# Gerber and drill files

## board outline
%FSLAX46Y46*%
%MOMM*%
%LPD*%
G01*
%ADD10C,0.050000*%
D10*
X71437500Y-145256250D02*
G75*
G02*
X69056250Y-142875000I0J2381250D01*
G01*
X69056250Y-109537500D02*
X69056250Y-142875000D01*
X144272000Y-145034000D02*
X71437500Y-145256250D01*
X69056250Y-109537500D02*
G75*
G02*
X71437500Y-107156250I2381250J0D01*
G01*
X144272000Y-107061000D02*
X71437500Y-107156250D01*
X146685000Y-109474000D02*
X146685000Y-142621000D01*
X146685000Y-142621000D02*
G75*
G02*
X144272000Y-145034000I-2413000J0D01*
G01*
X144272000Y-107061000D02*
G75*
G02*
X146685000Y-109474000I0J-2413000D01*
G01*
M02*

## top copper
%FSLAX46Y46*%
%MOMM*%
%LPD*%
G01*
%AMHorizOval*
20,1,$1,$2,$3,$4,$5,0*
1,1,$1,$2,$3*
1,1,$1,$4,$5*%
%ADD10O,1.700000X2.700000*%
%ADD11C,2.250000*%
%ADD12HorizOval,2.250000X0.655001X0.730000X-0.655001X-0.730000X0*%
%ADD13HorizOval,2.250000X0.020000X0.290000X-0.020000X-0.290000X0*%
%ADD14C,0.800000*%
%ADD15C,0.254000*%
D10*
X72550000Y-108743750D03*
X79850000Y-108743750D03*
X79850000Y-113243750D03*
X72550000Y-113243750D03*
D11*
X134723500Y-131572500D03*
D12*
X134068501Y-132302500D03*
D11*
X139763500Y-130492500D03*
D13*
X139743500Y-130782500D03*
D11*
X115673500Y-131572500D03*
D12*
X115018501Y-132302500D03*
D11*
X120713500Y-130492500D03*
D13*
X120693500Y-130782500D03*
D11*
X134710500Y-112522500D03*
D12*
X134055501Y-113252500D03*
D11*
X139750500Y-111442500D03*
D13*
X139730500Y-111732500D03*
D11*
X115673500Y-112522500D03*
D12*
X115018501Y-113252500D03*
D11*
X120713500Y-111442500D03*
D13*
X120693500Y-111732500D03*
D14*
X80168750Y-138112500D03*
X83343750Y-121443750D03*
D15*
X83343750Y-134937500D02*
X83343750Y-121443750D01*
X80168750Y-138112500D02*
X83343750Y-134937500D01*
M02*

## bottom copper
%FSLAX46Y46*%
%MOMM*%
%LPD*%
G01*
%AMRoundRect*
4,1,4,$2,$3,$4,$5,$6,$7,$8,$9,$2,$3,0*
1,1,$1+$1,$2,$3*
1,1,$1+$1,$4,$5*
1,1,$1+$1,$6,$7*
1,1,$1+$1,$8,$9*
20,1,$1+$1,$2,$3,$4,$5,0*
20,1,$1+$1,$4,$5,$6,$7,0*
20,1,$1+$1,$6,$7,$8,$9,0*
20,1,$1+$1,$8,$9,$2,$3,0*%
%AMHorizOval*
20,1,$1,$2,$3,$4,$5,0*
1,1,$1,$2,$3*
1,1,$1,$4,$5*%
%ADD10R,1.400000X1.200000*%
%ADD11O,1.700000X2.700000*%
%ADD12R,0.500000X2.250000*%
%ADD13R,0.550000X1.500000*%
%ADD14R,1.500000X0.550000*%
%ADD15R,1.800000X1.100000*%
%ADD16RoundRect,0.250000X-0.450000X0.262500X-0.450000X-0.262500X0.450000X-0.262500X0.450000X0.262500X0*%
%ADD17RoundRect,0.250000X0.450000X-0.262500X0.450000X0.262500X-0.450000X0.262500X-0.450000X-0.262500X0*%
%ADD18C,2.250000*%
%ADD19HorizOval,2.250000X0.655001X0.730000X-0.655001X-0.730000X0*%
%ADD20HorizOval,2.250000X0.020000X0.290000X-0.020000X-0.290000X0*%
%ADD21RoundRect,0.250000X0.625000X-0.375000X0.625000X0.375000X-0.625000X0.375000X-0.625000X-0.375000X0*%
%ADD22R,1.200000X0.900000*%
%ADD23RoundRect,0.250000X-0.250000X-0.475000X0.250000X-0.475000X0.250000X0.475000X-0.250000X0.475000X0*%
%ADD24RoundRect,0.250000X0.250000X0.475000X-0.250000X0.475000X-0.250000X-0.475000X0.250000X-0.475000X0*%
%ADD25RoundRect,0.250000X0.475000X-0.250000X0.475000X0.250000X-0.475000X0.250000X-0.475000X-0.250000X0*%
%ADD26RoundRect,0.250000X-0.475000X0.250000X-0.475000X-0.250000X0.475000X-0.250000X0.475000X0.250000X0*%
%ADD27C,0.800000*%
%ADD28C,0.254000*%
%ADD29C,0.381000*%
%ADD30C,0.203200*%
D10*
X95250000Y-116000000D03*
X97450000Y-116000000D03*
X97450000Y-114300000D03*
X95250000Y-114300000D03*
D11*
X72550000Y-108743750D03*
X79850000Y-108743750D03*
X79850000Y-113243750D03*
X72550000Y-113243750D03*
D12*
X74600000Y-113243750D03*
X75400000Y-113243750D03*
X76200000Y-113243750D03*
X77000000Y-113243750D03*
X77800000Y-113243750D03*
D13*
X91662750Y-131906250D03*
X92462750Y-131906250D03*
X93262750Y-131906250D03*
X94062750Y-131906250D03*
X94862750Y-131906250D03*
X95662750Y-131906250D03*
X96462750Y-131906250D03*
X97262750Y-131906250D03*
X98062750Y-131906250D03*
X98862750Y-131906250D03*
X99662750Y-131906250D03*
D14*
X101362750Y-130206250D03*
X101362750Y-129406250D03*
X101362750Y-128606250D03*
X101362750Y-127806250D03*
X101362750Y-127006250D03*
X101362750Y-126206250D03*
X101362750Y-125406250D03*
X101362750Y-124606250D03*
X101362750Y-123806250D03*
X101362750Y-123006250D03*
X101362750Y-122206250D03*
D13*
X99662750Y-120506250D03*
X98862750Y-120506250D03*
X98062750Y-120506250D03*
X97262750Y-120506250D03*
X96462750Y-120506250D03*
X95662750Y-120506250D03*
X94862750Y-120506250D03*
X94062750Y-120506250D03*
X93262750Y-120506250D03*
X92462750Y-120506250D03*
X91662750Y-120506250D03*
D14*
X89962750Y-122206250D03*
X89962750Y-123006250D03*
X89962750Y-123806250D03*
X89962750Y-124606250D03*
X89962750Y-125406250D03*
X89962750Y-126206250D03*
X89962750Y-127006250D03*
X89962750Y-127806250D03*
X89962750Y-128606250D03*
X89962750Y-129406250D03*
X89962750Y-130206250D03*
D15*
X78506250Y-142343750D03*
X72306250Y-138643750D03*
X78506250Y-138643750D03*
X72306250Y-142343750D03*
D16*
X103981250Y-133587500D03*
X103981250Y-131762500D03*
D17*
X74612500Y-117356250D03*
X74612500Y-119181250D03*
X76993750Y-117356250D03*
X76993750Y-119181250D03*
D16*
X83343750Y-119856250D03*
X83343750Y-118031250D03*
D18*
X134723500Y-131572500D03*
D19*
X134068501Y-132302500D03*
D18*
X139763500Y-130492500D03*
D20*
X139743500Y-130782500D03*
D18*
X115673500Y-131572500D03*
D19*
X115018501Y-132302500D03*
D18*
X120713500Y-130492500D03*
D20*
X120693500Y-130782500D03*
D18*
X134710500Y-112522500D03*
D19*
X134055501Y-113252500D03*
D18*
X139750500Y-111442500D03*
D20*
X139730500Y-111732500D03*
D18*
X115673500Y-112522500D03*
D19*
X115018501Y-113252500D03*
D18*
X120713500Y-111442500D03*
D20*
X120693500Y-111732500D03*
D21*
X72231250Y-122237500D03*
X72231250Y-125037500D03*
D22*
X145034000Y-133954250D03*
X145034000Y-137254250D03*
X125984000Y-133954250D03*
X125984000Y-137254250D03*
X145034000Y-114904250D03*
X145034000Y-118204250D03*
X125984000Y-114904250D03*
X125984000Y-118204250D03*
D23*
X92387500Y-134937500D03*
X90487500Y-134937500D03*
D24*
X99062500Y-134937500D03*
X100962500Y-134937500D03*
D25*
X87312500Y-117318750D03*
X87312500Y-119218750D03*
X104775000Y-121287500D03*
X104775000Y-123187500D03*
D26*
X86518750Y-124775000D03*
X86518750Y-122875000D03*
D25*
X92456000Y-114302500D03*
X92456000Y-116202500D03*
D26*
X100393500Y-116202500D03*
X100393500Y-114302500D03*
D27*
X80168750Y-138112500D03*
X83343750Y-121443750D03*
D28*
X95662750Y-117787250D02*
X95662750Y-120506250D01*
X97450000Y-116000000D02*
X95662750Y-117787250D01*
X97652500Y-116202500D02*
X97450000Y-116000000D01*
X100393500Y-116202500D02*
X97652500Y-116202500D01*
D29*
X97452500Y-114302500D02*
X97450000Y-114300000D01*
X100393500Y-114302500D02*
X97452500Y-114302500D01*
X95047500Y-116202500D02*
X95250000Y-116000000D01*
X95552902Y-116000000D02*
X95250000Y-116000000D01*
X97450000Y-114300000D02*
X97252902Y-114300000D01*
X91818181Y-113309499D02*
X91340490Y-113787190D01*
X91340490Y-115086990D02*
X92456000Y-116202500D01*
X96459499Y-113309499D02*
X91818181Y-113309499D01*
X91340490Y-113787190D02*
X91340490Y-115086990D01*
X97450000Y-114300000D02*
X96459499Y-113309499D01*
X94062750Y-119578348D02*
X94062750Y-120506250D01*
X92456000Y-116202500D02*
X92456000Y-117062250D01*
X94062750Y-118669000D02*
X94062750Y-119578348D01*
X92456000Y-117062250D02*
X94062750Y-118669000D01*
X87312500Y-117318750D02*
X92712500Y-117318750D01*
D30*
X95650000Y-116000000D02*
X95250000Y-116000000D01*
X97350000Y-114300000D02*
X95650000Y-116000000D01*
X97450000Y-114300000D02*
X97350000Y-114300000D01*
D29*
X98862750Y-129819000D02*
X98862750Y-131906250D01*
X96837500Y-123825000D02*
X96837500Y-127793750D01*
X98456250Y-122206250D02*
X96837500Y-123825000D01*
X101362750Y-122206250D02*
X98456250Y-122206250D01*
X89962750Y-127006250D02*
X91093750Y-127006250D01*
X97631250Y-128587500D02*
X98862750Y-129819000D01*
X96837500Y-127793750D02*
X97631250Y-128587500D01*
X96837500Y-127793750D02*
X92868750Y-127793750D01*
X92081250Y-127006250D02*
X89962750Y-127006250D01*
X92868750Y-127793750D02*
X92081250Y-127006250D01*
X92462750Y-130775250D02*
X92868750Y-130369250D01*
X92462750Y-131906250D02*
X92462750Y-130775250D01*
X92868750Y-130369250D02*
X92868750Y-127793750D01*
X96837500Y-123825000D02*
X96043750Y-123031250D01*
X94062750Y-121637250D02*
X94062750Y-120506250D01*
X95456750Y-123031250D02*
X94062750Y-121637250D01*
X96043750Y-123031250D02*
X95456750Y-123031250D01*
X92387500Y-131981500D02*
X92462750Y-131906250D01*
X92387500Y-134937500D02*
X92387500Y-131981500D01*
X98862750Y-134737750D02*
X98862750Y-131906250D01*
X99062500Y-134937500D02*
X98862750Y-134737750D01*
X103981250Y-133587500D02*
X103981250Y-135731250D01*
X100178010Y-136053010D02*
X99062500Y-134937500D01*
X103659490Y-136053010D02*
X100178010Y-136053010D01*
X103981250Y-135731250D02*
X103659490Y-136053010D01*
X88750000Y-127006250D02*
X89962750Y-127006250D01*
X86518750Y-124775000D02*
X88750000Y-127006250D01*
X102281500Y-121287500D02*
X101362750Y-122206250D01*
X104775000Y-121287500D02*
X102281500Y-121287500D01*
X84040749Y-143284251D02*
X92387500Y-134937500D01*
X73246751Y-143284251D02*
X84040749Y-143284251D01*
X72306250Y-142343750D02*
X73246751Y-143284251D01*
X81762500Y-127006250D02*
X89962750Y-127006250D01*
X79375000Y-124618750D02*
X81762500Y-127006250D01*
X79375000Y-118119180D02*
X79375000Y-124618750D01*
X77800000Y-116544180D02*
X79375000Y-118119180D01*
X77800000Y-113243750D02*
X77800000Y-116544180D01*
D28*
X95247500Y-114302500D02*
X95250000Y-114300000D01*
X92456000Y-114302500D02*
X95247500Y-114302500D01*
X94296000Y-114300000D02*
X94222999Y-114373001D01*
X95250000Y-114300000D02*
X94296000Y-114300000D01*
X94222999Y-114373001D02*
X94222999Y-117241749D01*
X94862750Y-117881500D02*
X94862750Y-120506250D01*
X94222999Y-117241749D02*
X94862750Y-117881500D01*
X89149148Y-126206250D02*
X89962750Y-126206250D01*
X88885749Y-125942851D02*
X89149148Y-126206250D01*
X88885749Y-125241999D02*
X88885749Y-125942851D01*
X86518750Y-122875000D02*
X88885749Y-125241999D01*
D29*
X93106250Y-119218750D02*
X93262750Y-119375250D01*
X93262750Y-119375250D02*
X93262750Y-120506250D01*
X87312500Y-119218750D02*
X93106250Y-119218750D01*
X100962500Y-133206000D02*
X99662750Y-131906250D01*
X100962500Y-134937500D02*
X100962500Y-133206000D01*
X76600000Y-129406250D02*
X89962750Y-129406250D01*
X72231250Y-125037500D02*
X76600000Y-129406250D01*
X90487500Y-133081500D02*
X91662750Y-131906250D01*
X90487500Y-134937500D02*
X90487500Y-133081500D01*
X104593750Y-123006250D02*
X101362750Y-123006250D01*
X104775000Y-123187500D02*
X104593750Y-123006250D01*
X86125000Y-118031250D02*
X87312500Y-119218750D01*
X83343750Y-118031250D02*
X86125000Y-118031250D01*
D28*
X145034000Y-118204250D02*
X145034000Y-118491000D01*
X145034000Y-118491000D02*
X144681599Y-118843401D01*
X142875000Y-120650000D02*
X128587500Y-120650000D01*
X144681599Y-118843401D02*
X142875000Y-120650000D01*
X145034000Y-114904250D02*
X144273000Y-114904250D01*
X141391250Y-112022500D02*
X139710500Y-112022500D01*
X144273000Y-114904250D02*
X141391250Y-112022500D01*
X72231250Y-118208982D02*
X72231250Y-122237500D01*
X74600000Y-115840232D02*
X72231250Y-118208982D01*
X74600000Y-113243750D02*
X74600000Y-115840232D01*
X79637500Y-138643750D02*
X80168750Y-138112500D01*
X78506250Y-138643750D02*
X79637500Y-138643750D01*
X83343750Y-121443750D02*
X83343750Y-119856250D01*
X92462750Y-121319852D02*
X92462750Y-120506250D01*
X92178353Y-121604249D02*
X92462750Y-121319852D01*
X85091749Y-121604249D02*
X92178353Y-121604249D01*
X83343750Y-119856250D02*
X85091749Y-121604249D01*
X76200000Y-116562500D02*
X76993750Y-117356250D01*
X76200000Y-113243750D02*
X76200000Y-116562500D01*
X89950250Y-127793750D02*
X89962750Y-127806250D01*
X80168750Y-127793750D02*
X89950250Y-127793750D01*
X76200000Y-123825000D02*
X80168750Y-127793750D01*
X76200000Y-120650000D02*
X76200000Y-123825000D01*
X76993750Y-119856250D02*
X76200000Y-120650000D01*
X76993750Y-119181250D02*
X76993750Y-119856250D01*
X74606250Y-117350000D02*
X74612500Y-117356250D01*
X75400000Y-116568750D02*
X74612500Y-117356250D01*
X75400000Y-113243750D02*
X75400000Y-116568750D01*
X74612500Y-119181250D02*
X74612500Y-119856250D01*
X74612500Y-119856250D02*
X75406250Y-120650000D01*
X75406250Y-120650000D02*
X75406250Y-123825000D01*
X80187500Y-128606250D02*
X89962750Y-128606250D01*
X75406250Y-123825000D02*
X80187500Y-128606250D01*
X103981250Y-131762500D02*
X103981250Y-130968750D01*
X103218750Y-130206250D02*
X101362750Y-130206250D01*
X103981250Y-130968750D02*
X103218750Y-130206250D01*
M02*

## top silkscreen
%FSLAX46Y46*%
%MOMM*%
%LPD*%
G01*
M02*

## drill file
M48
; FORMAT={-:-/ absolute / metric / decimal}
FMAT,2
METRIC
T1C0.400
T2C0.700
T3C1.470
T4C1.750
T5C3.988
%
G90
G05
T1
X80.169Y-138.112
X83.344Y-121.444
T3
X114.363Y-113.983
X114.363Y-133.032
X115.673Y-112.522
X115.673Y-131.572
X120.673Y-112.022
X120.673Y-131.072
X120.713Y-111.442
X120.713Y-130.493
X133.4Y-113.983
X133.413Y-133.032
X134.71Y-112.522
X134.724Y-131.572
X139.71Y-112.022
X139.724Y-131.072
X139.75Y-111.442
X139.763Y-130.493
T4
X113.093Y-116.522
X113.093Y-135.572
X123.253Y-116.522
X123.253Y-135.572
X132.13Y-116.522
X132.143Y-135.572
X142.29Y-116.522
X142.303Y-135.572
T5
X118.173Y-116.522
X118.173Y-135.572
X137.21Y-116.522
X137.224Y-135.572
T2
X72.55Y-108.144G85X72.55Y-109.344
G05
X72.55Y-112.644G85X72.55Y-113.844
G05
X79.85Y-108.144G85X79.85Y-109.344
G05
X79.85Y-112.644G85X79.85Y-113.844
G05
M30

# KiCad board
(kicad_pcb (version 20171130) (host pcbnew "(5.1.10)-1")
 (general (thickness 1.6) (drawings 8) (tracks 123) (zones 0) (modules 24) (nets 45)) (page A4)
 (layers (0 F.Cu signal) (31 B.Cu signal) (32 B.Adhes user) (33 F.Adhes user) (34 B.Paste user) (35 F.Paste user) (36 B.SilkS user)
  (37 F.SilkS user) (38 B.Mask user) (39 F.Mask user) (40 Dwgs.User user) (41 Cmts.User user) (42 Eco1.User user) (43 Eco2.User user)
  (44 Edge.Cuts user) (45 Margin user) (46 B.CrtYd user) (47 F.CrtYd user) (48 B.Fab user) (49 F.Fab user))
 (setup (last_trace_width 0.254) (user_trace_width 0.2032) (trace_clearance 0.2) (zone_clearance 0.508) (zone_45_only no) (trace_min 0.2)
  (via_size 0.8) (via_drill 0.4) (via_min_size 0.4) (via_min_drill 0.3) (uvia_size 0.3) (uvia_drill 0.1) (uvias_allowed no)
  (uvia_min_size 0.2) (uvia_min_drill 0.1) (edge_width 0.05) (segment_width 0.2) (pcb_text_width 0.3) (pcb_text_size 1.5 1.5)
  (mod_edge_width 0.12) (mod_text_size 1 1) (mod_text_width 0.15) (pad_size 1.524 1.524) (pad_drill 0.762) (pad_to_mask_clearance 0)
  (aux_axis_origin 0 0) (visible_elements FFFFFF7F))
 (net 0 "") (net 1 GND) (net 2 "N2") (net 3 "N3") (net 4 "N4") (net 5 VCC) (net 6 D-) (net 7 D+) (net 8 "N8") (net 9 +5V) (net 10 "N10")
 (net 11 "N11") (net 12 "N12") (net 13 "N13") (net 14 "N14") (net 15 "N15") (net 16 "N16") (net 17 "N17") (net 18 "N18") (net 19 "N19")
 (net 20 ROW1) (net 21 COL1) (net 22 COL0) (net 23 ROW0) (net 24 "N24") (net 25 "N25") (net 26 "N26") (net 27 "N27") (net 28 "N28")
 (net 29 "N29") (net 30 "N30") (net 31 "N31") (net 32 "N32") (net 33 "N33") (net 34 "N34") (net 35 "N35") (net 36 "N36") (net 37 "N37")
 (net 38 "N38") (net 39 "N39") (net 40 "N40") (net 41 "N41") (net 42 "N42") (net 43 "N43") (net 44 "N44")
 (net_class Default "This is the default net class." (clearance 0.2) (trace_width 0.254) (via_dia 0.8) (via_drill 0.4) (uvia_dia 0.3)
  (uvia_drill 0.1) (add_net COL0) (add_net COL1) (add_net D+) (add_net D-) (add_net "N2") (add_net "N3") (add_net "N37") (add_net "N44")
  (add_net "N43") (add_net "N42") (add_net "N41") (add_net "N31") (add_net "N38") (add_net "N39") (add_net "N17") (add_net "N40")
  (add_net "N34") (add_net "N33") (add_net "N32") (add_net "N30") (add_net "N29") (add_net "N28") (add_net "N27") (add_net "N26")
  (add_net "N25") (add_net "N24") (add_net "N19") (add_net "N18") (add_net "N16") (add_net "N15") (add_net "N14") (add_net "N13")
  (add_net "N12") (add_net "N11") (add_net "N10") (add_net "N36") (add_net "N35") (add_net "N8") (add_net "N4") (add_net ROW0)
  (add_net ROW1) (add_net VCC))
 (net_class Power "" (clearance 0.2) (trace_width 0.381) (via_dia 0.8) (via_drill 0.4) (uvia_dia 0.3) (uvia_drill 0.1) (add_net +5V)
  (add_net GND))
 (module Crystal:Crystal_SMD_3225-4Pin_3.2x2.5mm (layer B.Cu) (at 96.35 115.15)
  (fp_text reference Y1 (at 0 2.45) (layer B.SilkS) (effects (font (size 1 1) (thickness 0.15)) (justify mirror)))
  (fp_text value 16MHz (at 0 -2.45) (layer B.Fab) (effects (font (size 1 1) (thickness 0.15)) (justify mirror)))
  (pad 4 smd rect (at -1.1 0.85) (size 1.4 1.2) (layers B.Cu B.Paste B.Mask) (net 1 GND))
  (pad 3 smd rect (at 1.1 0.85) (size 1.4 1.2) (layers B.Cu B.Paste B.Mask) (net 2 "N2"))
  (pad 2 smd rect (at 1.1 -0.85) (size 1.4 1.2) (layers B.Cu B.Paste B.Mask) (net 1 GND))
  (pad 1 smd rect (at -1.1 -0.85) (size 1.4 1.2) (layers B.Cu B.Paste B.Mask) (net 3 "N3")))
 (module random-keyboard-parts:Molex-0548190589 (layer B.Cu) (at 76.2 108.74375 270)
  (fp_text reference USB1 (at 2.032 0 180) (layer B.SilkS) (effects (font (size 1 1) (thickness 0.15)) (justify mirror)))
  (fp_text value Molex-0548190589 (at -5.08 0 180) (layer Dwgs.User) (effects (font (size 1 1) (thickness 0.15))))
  (pad 6 thru_hole oval (at 0 3.65 270) (size 2.7 1.7) (drill oval 1.9 0.7) (layers *.Cu *.Mask) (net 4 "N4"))
  (pad 6 thru_hole oval (at 0 -3.65 270) (size 2.7 1.7) (drill oval 1.9 0.7) (layers *.Cu *.Mask) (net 4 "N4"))
  (pad 6 thru_hole oval (at 4.5 -3.65 270) (size 2.7 1.7) (drill oval 1.9 0.7) (layers *.Cu *.Mask) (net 4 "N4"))
  (pad 6 thru_hole oval (at 4.5 3.65 270) (size 2.7 1.7) (drill oval 1.9 0.7) (layers *.Cu *.Mask) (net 4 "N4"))
  (pad 5 smd rect (at 4.5 1.6 270) (size 2.25 0.5) (layers B.Cu B.Paste B.Mask) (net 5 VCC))
  (pad 4 smd rect (at 4.5 0.8 270) (size 2.25 0.5) (layers B.Cu B.Paste B.Mask) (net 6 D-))
  (pad 3 smd rect (at 4.5 0 270) (size 2.25 0.5) (layers B.Cu B.Paste B.Mask) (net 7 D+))
  (pad 2 smd rect (at 4.5 -0.8 270) (size 2.25 0.5) (layers B.Cu B.Paste B.Mask) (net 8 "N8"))
  (pad 1 smd rect (at 4.5 -1.6 270) (size 2.25 0.5) (layers B.Cu B.Paste B.Mask) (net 1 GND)))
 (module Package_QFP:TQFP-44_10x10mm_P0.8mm (layer B.Cu) (at 95.66275 126.20625)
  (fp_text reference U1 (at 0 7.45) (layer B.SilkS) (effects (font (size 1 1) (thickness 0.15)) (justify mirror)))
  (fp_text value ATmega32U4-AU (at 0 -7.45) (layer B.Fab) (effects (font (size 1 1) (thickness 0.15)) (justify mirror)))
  (pad 44 smd rect (at -4 5.7 270) (size 1.5 0.55) (layers B.Cu B.Paste B.Mask) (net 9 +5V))
  (pad 43 smd rect (at -3.2 5.7 270) (size 1.5 0.55) (layers B.Cu B.Paste B.Mask) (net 1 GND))
  (pad 42 smd rect (at -2.4 5.7 270) (size 1.5 0.55) (layers B.Cu B.Paste B.Mask) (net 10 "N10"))
  (pad 41 smd rect (at -1.6 5.7 270) (size 1.5 0.55) (layers B.Cu B.Paste B.Mask) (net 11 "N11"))
  (pad 40 smd rect (at -0.8 5.7 270) (size 1.5 0.55) (layers B.Cu B.Paste B.Mask) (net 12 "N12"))
  (pad 39 smd rect (at 0 5.7 270) (size 1.5 0.55) (layers B.Cu B.Paste B.Mask) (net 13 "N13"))
  (pad 38 smd rect (at 0.8 5.7 270) (size 1.5 0.55) (layers B.Cu B.Paste B.Mask) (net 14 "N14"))
  (pad 37 smd rect (at 1.6 5.7 270) (size 1.5 0.55) (layers B.Cu B.Paste B.Mask) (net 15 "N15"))
  (pad 36 smd rect (at 2.4 5.7 270) (size 1.5 0.55) (layers B.Cu B.Paste B.Mask) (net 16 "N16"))
  (pad 35 smd rect (at 3.2 5.7 270) (size 1.5 0.55) (layers B.Cu B.Paste B.Mask) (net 1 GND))
  (pad 34 smd rect (at 4 5.7 270) (size 1.5 0.55) (layers B.Cu B.Paste B.Mask) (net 9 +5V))
  (pad 33 smd rect (at 5.7 4) (size 1.5 0.55) (layers B.Cu B.Paste B.Mask) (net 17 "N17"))
  (pad 32 smd rect (at 5.7 3.2) (size 1.5 0.55) (layers B.Cu B.Paste B.Mask) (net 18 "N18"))
  (pad 31 smd rect (at 5.7 2.4) (size 1.5 0.55) (layers B.Cu B.Paste B.Mask) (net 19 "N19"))
  (pad 30 smd rect (at 5.7 1.6) (size 1.5 0.55) (layers B.Cu B.Paste B.Mask) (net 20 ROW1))
  (pad 29 smd rect (at 5.7 0.8) (size 1.5 0.55) (layers B.Cu B.Paste B.Mask) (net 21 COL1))
  (pad 28 smd rect (at 5.7 0) (size 1.5 0.55) (layers B.Cu B.Paste B.Mask) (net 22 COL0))
  (pad 27 smd rect (at 5.7 -0.8) (size 1.5 0.55) (layers B.Cu B.Paste B.Mask) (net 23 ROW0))
  (pad 26 smd rect (at 5.7 -1.6) (size 1.5 0.55) (layers B.Cu B.Paste B.Mask) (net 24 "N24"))
  (pad 25 smd rect (at 5.7 -2.4) (size 1.5 0.55) (layers B.Cu B.Paste B.Mask) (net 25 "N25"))
  (pad 24 smd rect (at 5.7 -3.2) (size 1.5 0.55) (layers B.Cu B.Paste B.Mask) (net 9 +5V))
  (pad 23 smd rect (at 5.7 -4) (size 1.5 0.55) (layers B.Cu B.Paste B.Mask) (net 1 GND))
  (pad 22 smd rect (at 4 -5.7 270) (size 1.5 0.55) (layers B.Cu B.Paste B.Mask) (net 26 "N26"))
  (pad 21 smd rect (at 3.2 -5.7 270) (size 1.5 0.55) (layers B.Cu B.Paste B.Mask) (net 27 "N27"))
  (pad 20 smd rect (at 2.4 -5.7 270) (size 1.5 0.55) (layers B.Cu B.Paste B.Mask) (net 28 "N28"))
  (pad 19 smd rect (at 1.6 -5.7 270) (size 1.5 0.55) (layers B.Cu B.Paste B.Mask) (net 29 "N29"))
  (pad 18 smd rect (at 0.8 -5.7 270) (size 1.5 0.55) (layers B.Cu B.Paste B.Mask) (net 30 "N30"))
  (pad 17 smd rect (at 0 -5.7 270) (size 1.5 0.55) (layers B.Cu B.Paste B.Mask) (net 2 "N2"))
  (pad 16 smd rect (at -0.8 -5.7 270) (size 1.5 0.55) (layers B.Cu B.Paste B.Mask) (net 3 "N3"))
  (pad 15 smd rect (at -1.6 -5.7 270) (size 1.5 0.55) (layers B.Cu B.Paste B.Mask) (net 1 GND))
  (pad 14 smd rect (at -2.4 -5.7 270) (size 1.5 0.55) (layers B.Cu B.Paste B.Mask) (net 9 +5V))
  (pad 13 smd rect (at -3.2 -5.7 270) (size 1.5 0.55) (layers B.Cu B.Paste B.Mask) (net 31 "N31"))
  (pad 12 smd rect (at -4 -5.7 270) (size 1.5 0.55) (layers B.Cu B.Paste B.Mask) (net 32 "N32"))
  (pad 11 smd rect (at -5.7 -4) (size 1.5 0.55) (layers B.Cu B.Paste B.Mask) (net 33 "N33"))
  (pad 10 smd rect (at -5.7 -3.2) (size 1.5 0.55) (layers B.Cu B.Paste B.Mask) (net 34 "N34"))
  (pad 9 smd rect (at -5.7 -2.4) (size 1.5 0.55) (layers B.Cu B.Paste B.Mask) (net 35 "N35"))
  (pad 8 smd rect (at -5.7 -1.6) (size 1.5 0.55) (layers B.Cu B.Paste B.Mask) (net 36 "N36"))
  (pad 7 smd rect (at -5.7 -0.8) (size 1.5 0.55) (layers B.Cu B.Paste B.Mask) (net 9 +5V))
  (pad 6 smd rect (at -5.7 0) (size 1.5 0.55) (layers B.Cu B.Paste B.Mask) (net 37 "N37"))
  (pad 5 smd rect (at -5.7 0.8) (size 1.5 0.55) (layers B.Cu B.Paste B.Mask) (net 1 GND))
  (pad 4 smd rect (at -5.7 1.6) (size 1.5 0.55) (layers B.Cu B.Paste B.Mask) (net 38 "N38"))
  (pad 3 smd rect (at -5.7 2.4) (size 1.5 0.55) (layers B.Cu B.Paste B.Mask) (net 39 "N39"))
  (pad 2 smd rect (at -5.7 3.2) (size 1.5 0.55) (layers B.Cu B.Paste B.Mask) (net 9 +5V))
  (pad 1 smd rect (at -5.7 4) (size 1.5 0.55) (layers B.Cu B.Paste B.Mask) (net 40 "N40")))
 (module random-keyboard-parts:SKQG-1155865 (layer B.Cu) (at 75.40625 140.49375 180)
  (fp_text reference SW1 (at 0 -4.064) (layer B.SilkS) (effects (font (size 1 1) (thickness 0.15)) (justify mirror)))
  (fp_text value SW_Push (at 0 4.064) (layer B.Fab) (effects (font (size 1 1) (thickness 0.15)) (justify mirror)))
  (pad 4 smd rect (at -3.1 -1.85 180) (size 1.8 1.1) (layers B.Cu B.Paste B.Mask))
  (pad 3 smd rect (at 3.1 1.85 180) (size 1.8 1.1) (layers B.Cu B.Paste B.Mask))
  (pad 2 smd rect (at -3.1 1.85 180) (size 1.8 1.1) (layers B.Cu B.Paste B.Mask) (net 31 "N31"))
  (pad 1 smd rect (at 3.1 -1.85 180) (size 1.8 1.1) (layers B.Cu B.Paste B.Mask) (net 1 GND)))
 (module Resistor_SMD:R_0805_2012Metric (layer B.Cu) (at 103.98125 132.675 270)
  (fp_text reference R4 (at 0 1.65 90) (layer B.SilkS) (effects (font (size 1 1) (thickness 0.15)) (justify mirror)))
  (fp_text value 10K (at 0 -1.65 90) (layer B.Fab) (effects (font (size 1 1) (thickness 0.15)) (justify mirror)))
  (pad 2 smd roundrect (at 0.9125 0 270) (size 1.025 1.4) (layers B.Cu B.Paste B.Mask) (roundrect_rratio 0.243902) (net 1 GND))
  (pad 1 smd roundrect (at -0.9125 0 270) (size 1.025 1.4) (layers B.Cu B.Paste B.Mask) (roundrect_rratio 0.243902) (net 17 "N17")))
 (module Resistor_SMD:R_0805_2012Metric (layer B.Cu) (at 74.6125 118.26875 90)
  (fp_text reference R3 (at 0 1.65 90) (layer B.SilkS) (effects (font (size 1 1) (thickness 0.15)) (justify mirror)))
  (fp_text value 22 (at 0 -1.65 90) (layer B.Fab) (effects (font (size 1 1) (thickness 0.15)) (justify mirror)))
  (pad 2 smd roundrect (at 0.9125 0 90) (size 1.025 1.4) (layers B.Cu B.Paste B.Mask) (roundrect_rratio 0.243902) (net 6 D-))
  (pad 1 smd roundrect (at -0.9125 0 90) (size 1.025 1.4) (layers B.Cu B.Paste B.Mask) (roundrect_rratio 0.243902) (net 39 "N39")))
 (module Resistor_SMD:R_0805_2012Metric (layer B.Cu) (at 76.99375 118.26875 90)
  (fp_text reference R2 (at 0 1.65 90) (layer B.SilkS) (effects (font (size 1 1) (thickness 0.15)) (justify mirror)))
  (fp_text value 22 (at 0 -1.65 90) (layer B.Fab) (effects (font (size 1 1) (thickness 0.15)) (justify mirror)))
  (pad 2 smd roundrect (at 0.9125 0 90) (size 1.025 1.4) (layers B.Cu B.Paste B.Mask) (roundrect_rratio 0.243902) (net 7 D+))
  (pad 1 smd roundrect (at -0.9125 0 90) (size 1.025 1.4) (layers B.Cu B.Paste B.Mask) (roundrect_rratio 0.243902) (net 38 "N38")))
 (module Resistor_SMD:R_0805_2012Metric (layer B.Cu) (at 83.34375 118.94375 270)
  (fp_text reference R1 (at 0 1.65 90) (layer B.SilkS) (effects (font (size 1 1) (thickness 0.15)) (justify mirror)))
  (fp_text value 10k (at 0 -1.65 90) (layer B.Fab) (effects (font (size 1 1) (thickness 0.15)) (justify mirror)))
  (pad 2 smd roundrect (at 0.9125 0 270) (size 1.025 1.4) (layers B.Cu B.Paste B.Mask) (roundrect_rratio 0.243902) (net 31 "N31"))
  (pad 1 smd roundrect (at -0.9125 0 270) (size 1.025 1.4) (layers B.Cu B.Paste B.Mask) (roundrect_rratio 0.243902) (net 9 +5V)))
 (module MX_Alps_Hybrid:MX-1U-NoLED (layer F.Cu) (at 137.2235 135.5725)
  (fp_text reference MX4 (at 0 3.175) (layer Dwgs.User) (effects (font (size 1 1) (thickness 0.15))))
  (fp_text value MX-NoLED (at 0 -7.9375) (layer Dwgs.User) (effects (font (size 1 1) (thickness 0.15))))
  (pad "" np_thru_hole circle (at 5.08 0 48.0996) (size 1.75 1.75) (drill 1.75) (layers *.Cu *.Mask))
  (pad "" np_thru_hole circle (at -5.08 0 48.0996) (size 1.75 1.75) (drill 1.75) (layers *.Cu *.Mask))
  (pad 1 thru_hole circle (at -2.5 -4) (size 2.25 2.25) (drill 1.47) (layers *.Cu B.Mask) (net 21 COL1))
  (pad "" np_thru_hole circle (at 0 0) (size 3.9878 3.9878) (drill 3.9878) (layers *.Cu *.Mask))
  (pad 1 thru_hole oval (at -3.81 -2.54 48.0996) (size 4.211556 2.25) (drill 1.47 (offset 0.980778 0)) (layers *.Cu B.Mask) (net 21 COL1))
  (pad 2 thru_hole circle (at 2.54 -5.08) (size 2.25 2.25) (drill 1.47) (layers *.Cu B.Mask) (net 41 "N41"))
  (pad 2 thru_hole oval (at 2.5 -4.5 86.0548) (size 2.831378 2.25) (drill 1.47 (offset 0.290689 0)) (layers *.Cu B.Mask) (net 41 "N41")))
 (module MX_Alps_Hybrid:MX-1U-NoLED (layer F.Cu) (at 118.1735 135.5725)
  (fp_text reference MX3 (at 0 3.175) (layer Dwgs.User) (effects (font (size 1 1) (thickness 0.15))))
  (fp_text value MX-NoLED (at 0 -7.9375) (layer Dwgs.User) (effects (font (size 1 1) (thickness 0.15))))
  (pad "" np_thru_hole circle (at 5.08 0 48.0996) (size 1.75 1.75) (drill 1.75) (layers *.Cu *.Mask))
  (pad "" np_thru_hole circle (at -5.08 0 48.0996) (size 1.75 1.75) (drill 1.75) (layers *.Cu *.Mask))
  (pad 1 thru_hole circle (at -2.5 -4) (size 2.25 2.25) (drill 1.47) (layers *.Cu B.Mask) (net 22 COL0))
  (pad "" np_thru_hole circle (at 0 0) (size 3.9878 3.9878) (drill 3.9878) (layers *.Cu *.Mask))
  (pad 1 thru_hole oval (at -3.81 -2.54 48.0996) (size 4.211556 2.25) (drill 1.47 (offset 0.980778 0)) (layers *.Cu B.Mask) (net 22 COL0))
  (pad 2 thru_hole circle (at 2.54 -5.08) (size 2.25 2.25) (drill 1.47) (layers *.Cu B.Mask) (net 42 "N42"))
  (pad 2 thru_hole oval (at 2.5 -4.5 86.0548) (size 2.831378 2.25) (drill 1.47 (offset 0.290689 0)) (layers *.Cu B.Mask) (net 42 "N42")))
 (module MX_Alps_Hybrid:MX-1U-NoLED (layer F.Cu) (at 137.2105 116.5225)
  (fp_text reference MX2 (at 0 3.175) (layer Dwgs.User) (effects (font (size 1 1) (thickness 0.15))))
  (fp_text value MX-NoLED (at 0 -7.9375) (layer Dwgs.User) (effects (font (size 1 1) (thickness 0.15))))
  (pad "" np_thru_hole circle (at 5.08 0 48.0996) (size 1.75 1.75) (drill 1.75) (layers *.Cu *.Mask))
  (pad "" np_thru_hole circle (at -5.08 0 48.0996) (size 1.75 1.75) (drill 1.75) (layers *.Cu *.Mask))
  (pad 1 thru_hole circle (at -2.5 -4) (size 2.25 2.25) (drill 1.47) (layers *.Cu B.Mask) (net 21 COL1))
  (pad "" np_thru_hole circle (at 0 0) (size 3.9878 3.9878) (drill 3.9878) (layers *.Cu *.Mask))
  (pad 1 thru_hole oval (at -3.81 -2.54 48.0996) (size 4.211556 2.25) (drill 1.47 (offset 0.980778 0)) (layers *.Cu B.Mask) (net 21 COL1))
  (pad 2 thru_hole circle (at 2.54 -5.08) (size 2.25 2.25) (drill 1.47) (layers *.Cu B.Mask) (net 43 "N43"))
  (pad 2 thru_hole oval (at 2.5 -4.5 86.0548) (size 2.831378 2.25) (drill 1.47 (offset 0.290689 0)) (layers *.Cu B.Mask) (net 43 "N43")))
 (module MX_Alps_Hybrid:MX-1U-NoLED (layer F.Cu) (at 118.1735 116.5225)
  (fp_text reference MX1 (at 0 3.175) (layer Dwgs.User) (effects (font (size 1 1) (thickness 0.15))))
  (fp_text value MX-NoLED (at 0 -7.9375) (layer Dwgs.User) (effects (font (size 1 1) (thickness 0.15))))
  (pad "" np_thru_hole circle (at 5.08 0 48.0996) (size 1.75 1.75) (drill 1.75) (layers *.Cu *.Mask))
  (pad "" np_thru_hole circle (at -5.08 0 48.0996) (size 1.75 1.75) (drill 1.75) (layers *.Cu *.Mask))
  (pad 1 thru_hole circle (at -2.5 -4) (size 2.25 2.25) (drill 1.47) (layers *.Cu B.Mask) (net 22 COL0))
  (pad "" np_thru_hole circle (at 0 0) (size 3.9878 3.9878) (drill 3.9878) (layers *.Cu *.Mask))
  (pad 1 thru_hole oval (at -3.81 -2.54 48.0996) (size 4.211556 2.25) (drill 1.47 (offset 0.980778 0)) (layers *.Cu B.Mask) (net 22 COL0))
  (pad 2 thru_hole circle (at 2.54 -5.08) (size 2.25 2.25) (drill 1.47) (layers *.Cu B.Mask) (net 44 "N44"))
  (pad 2 thru_hole oval (at 2.5 -4.5 86.0548) (size 2.831378 2.25) (drill 1.47 (offset 0.290689 0)) (layers *.Cu B.Mask) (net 44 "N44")))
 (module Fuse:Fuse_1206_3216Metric (layer B.Cu) (at 72.23125 123.6375 90)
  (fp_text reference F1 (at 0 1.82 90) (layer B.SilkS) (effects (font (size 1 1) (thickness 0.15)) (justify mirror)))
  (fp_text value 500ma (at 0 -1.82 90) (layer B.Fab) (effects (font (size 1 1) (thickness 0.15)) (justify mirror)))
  (pad 2 smd roundrect (at 1.4 0 90) (size 1.25 1.75) (layers B.Cu B.Paste B.Mask) (roundrect_rratio 0.2) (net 5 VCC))
  (pad 1 smd roundrect (at -1.4 0 90) (size 1.25 1.75) (layers B.Cu B.Paste B.Mask) (roundrect_rratio 0.2) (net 9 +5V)))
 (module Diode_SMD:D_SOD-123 (layer B.Cu) (at 145.034 135.60425 90)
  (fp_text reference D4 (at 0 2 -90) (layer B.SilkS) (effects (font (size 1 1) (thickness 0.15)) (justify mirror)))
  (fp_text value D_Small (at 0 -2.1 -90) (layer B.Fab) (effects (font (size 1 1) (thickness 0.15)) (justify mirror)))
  (pad 2 smd rect (at 1.65 0 90) (size 0.9 1.2) (layers B.Cu B.Paste B.Mask) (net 41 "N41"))
  (pad 1 smd rect (at -1.65 0 90) (size 0.9 1.2) (layers B.Cu B.Paste B.Mask) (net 20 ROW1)))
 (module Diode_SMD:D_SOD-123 (layer B.Cu) (at 125.984 135.60425 90)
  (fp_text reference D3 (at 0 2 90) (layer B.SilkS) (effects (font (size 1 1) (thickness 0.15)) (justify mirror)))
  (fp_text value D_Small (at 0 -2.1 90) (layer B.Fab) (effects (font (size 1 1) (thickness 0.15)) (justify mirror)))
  (pad 2 smd rect (at 1.65 0 90) (size 0.9 1.2) (layers B.Cu B.Paste B.Mask) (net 42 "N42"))
  (pad 1 smd rect (at -1.65 0 90) (size 0.9 1.2) (layers B.Cu B.Paste B.Mask) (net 20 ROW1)))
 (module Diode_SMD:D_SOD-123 (layer B.Cu) (at 145.034 116.55425 90)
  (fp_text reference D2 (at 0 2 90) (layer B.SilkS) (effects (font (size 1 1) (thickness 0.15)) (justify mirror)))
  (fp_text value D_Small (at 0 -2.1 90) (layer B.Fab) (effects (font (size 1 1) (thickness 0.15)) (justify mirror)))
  (pad 2 smd rect (at 1.65 0 90) (size 0.9 1.2) (layers B.Cu B.Paste B.Mask) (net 43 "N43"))
  (pad 1 smd rect (at -1.65 0 90) (size 0.9 1.2) (layers B.Cu B.Paste B.Mask) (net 23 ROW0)))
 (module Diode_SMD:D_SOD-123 (layer B.Cu) (at 125.984 116.55425 90)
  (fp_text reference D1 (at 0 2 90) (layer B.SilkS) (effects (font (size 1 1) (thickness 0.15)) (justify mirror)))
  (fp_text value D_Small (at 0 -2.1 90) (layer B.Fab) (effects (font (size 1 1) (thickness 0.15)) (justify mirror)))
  (pad 2 smd rect (at 1.65 0 90) (size 0.9 1.2) (layers B.Cu B.Paste B.Mask) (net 44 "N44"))
  (pad 1 smd rect (at -1.65 0 90) (size 0.9 1.2) (layers B.Cu B.Paste B.Mask) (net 23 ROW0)))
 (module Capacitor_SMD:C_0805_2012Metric (layer B.Cu) (at 91.4375 134.9375)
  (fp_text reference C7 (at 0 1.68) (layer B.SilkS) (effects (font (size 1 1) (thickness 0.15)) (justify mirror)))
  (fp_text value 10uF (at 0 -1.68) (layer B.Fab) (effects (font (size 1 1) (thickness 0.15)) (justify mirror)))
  (pad 2 smd roundrect (at 0.95 0) (size 1 1.45) (layers B.Cu B.Paste B.Mask) (roundrect_rratio 0.25) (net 1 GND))
  (pad 1 smd roundrect (at -0.95 0) (size 1 1.45) (layers B.Cu B.Paste B.Mask) (roundrect_rratio 0.25) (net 9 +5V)))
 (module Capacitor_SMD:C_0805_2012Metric (layer B.Cu) (at 100.0125 134.9375 180)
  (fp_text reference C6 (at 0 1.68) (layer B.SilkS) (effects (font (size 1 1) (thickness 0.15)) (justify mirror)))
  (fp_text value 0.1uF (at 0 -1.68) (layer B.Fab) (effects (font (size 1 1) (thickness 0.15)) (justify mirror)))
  (pad 2 smd roundrect (at 0.95 0 180) (size 1 1.45) (layers B.Cu B.Paste B.Mask) (roundrect_rratio 0.25) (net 1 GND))
  (pad 1 smd roundrect (at -0.95 0 180) (size 1 1.45) (layers B.Cu B.Paste B.Mask) (roundrect_rratio 0.25) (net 9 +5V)))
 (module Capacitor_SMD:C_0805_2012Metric (layer B.Cu) (at 87.3125 118.26875 90)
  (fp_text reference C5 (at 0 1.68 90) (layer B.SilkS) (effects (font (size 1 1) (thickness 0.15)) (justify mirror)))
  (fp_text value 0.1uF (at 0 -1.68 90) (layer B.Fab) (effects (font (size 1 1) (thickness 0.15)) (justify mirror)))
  (pad 2 smd roundrect (at 0.95 0 90) (size 1 1.45) (layers B.Cu B.Paste B.Mask) (roundrect_rratio 0.25) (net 1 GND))
  (pad 1 smd roundrect (at -0.95 0 90) (size 1 1.45) (layers B.Cu B.Paste B.Mask) (roundrect_rratio 0.25) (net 9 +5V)))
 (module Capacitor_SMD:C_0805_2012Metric (layer B.Cu) (at 104.775 122.2375 90)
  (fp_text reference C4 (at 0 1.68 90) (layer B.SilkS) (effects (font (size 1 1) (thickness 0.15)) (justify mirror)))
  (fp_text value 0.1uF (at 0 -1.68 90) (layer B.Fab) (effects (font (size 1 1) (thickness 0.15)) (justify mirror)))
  (pad 2 smd roundrect (at 0.95 0 90) (size 1 1.45) (layers B.Cu B.Paste B.Mask) (roundrect_rratio 0.25) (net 1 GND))
  (pad 1 smd roundrect (at -0.95 0 90) (size 1 1.45) (layers B.Cu B.Paste B.Mask) (roundrect_rratio 0.25) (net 9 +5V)))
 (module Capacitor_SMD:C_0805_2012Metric (layer B.Cu) (at 86.51875 123.825 270)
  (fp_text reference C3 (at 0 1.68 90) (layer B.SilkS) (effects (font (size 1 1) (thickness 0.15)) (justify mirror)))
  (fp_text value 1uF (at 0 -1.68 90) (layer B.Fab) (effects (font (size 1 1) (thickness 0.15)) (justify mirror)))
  (pad 2 smd roundrect (at 0.95 0 270) (size 1 1.45) (layers B.Cu B.Paste B.Mask) (roundrect_rratio 0.25) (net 1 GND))
  (pad 1 smd roundrect (at -0.95 0 270) (size 1 1.45) (layers B.Cu B.Paste B.Mask) (roundrect_rratio 0.25) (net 37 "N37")))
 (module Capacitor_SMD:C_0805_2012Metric (layer B.Cu) (at 92.456 115.2525 90)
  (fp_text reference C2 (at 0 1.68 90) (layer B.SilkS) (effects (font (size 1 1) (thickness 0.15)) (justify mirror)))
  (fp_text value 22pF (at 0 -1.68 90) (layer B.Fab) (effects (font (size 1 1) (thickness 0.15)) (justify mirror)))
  (pad 2 smd roundrect (at 0.95 0 90) (size 1 1.45) (layers B.Cu B.Paste B.Mask) (roundrect_rratio 0.25) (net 3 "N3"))
  (pad 1 smd roundrect (at -0.95 0 90) (size 1 1.45) (layers B.Cu B.Paste B.Mask) (roundrect_rratio 0.25) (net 1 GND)))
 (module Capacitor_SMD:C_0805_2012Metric (layer B.Cu) (at 100.3935 115.2525 270)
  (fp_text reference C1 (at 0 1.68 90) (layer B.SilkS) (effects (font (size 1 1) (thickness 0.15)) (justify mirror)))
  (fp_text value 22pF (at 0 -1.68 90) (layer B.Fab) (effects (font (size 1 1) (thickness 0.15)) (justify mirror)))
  (pad 2 smd roundrect (at 0.95 0 270) (size 1 1.45) (layers B.Cu B.Paste B.Mask) (roundrect_rratio 0.25) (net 2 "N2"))
  (pad 1 smd roundrect (at -0.95 0 270) (size 1 1.45) (layers B.Cu B.Paste B.Mask) (roundrect_rratio 0.25) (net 1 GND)))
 (gr_arc (start 71.4375 142.875) (end 69.05625 142.875) (angle -90) (layer Edge.Cuts) (width 0.05))
 (gr_line (start 69.05625 109.5375) (end 69.05625 142.875) (layer Edge.Cuts) (width 0.05))
 (gr_line (start 144.272 145.034) (end 71.4375 145.25625) (layer Edge.Cuts) (width 0.05))
 (gr_arc (start 71.4375 109.5375) (end 71.4375 107.15625) (angle -90) (layer Edge.Cuts) (width 0.05))
 (gr_line (start 144.272 107.061) (end 71.4375 107.15625) (layer Edge.Cuts) (width 0.05))
 (gr_line (start 146.685 109.474) (end 146.685 142.621) (layer Edge.Cuts) (width 0.05))
 (gr_arc (start 144.272 142.621) (end 144.272 145.034) (angle -90) (layer Edge.Cuts) (width 0.05))
 (gr_arc (start 144.272 109.474) (end 146.685 109.474) (angle -90) (layer Edge.Cuts) (width 0.05))
 (segment (start 95.66275 117.78725) (end 95.66275 120.50625) (width 0.254) (layer B.Cu) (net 2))
 (segment (start 97.45 116) (end 95.66275 117.78725) (width 0.254) (layer B.Cu) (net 2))
 (segment (start 97.6525 116.2025) (end 97.45 116) (width 0.254) (layer B.Cu) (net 2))
 (segment (start 100.3935 116.2025) (end 97.6525 116.2025) (width 0.254) (layer B.Cu) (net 2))
 (segment (start 97.4525 114.3025) (end 97.45 114.3) (width 0.381) (layer B.Cu) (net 1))
 (segment (start 100.3935 114.3025) (end 97.4525 114.3025) (width 0.381) (layer B.Cu) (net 1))
 (segment (start 95.0475 116.2025) (end 95.25 116) (width 0.381) (layer B.Cu) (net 1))
 (segment (start 95.552902 116) (end 95.25 116) (width 0.381) (layer B.Cu) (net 1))
 (segment (start 97.45 114.3) (end 97.252902 114.3) (width 0.381) (layer B.Cu) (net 1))
 (segment (start 91.818181 113.309499) (end 91.34049 113.78719) (width 0.381) (layer B.Cu) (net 1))
 (segment (start 91.34049 115.08699) (end 92.456 116.2025) (width 0.381) (layer B.Cu) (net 1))
 (segment (start 96.459499 113.309499) (end 91.818181 113.309499) (width 0.381) (layer B.Cu) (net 1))
 (segment (start 91.34049 113.78719) (end 91.34049 115.08699) (width 0.381) (layer B.Cu) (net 1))
 (segment (start 97.45 114.3) (end 96.459499 113.309499) (width 0.381) (layer B.Cu) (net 1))
 (segment (start 94.06275 119.578348) (end 94.06275 120.50625) (width 0.381) (layer B.Cu) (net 1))
 (segment (start 92.456 116.2025) (end 92.456 117.06225) (width 0.381) (layer B.Cu) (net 1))
 (segment (start 94.06275 118.669) (end 94.06275 119.578348) (width 0.381) (layer B.Cu) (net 1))
 (segment (start 92.456 117.06225) (end 94.06275 118.669) (width 0.381) (layer B.Cu) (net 1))
 (segment (start 87.3125 117.31875) (end 92.7125 117.31875) (width 0.381) (layer B.Cu) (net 1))
 (segment (start 95.65 116) (end 95.25 116) (width 0.2032) (layer B.Cu) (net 1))
 (segment (start 97.35 114.3) (end 95.65 116) (width 0.2032) (layer B.Cu) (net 1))
 (segment (start 97.45 114.3) (end 97.35 114.3) (width 0.2032) (layer B.Cu) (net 1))
 (segment (start 98.86275 129.819) (end 98.86275 131.90625) (width 0.381) (layer B.Cu) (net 1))
 (segment (start 96.8375 123.825) (end 96.8375 127.79375) (width 0.381) (layer B.Cu) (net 1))
 (segment (start 98.45625 122.20625) (end 96.8375 123.825) (width 0.381) (layer B.Cu) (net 1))
 (segment (start 101.36275 122.20625) (end 98.45625 122.20625) (width 0.381) (layer B.Cu) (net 1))
 (segment (start 89.96275 127.00625) (end 91.09375 127.00625) (width 0.381) (layer B.Cu) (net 1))
 (segment (start 97.63125 128.5875) (end 98.86275 129.819) (width 0.381) (layer B.Cu) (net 1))
 (segment (start 96.8375 127.79375) (end 97.63125 128.5875) (width 0.381) (layer B.Cu) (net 1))
 (segment (start 96.8375 127.79375) (end 92.86875 127.79375) (width 0.381) (layer B.Cu) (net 1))
 (segment (start 92.08125 127.00625) (end 89.96275 127.00625) (width 0.381) (layer B.Cu) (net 1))
 (segment (start 92.86875 127.79375) (end 92.08125 127.00625) (width 0.381) (layer B.Cu) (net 1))
 (segment (start 92.46275 130.77525) (end 92.86875 130.36925) (width 0.381) (layer B.Cu) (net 1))
 (segment (start 92.46275 131.90625) (end 92.46275 130.77525) (width 0.381) (layer B.Cu) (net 1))
 (segment (start 92.86875 130.36925) (end 92.86875 127.79375) (width 0.381) (layer B.Cu) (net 1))
 (segment (start 96.8375 123.825) (end 96.04375 123.03125) (width 0.381) (layer B.Cu) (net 1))
 (segment (start 94.06275 121.63725) (end 94.06275 120.50625) (width 0.381) (layer B.Cu) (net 1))
 (segment (start 95.45675 123.03125) (end 94.06275 121.63725) (width 0.381) (layer B.Cu) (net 1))
 (segment (start 96.04375 123.03125) (end 95.45675 123.03125) (width 0.381) (layer B.Cu) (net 1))
 (segment (start 92.3875 131.9815) (end 92.46275 131.90625) (width 0.381) (layer B.Cu) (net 1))
 (segment (start 92.3875 134.9375) (end 92.3875 131.9815) (width 0.381) (layer B.Cu) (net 1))
 (segment (start 98.86275 134.73775) (end 98.86275 131.90625) (width 0.381) (layer B.Cu) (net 1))
 (segment (start 99.0625 134.9375) (end 98.86275 134.73775) (width 0.381) (layer B.Cu) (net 1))
 (segment (start 103.98125 133.5875) (end 103.98125 135.73125) (width 0.381) (layer B.Cu) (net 1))
 (segment (start 100.17801 136.05301) (end 99.0625 134.9375) (width 0.381) (layer B.Cu) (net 1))
 (segment (start 103.65949 136.05301) (end 100.17801 136.05301) (width 0.381) (layer B.Cu) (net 1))
 (segment (start 103.98125 135.73125) (end 103.65949 136.05301) (width 0.381) (layer B.Cu) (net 1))
 (segment (start 88.75 127.00625) (end 89.96275 127.00625) (width 0.381) (layer B.Cu) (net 1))
 (segment (start 86.51875 124.775) (end 88.75 127.00625) (width 0.381) (layer B.Cu) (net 1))
 (segment (start 102.2815 121.2875) (end 101.36275 122.20625) (width 0.381) (layer B.Cu) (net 1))
 (segment (start 104.775 121.2875) (end 102.2815 121.2875) (width 0.381) (layer B.Cu) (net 1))
 (segment (start 84.040749 143.284251) (end 92.3875 134.9375) (width 0.381) (layer B.Cu) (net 1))
 (segment (start 73.246751 143.284251) (end 84.040749 143.284251) (width 0.381) (layer B.Cu) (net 1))
 (segment (start 72.30625 142.34375) (end 73.246751 143.284251) (width 0.381) (layer B.Cu) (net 1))
 (segment (start 81.7625 127.00625) (end 89.96275 127.00625) (width 0.381) (layer B.Cu) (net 1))
 (segment (start 79.375 124.61875) (end 81.7625 127.00625) (width 0.381) (layer B.Cu) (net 1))
 (segment (start 79.375 118.11918) (end 79.375 124.61875) (width 0.381) (layer B.Cu) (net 1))
 (segment (start 77.8 116.54418) (end 79.375 118.11918) (width 0.381) (layer B.Cu) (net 1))
 (segment (start 77.8 113.24375) (end 77.8 116.54418) (width 0.381) (layer B.Cu) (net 1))
 (segment (start 95.2475 114.3025) (end 95.25 114.3) (width 0.254) (layer B.Cu) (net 3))
 (segment (start 92.456 114.3025) (end 95.2475 114.3025) (width 0.254) (layer B.Cu) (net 3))
 (segment (start 94.296 114.3) (end 94.222999 114.373001) (width 0.254) (layer B.Cu) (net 3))
 (segment (start 95.25 114.3) (end 94.296 114.3) (width 0.254) (layer B.Cu) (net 3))
 (segment (start 94.222999 114.373001) (end 94.222999 117.241749) (width 0.254) (layer B.Cu) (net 3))
 (segment (start 94.86275 117.8815) (end 94.86275 120.50625) (width 0.254) (layer B.Cu) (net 3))
 (segment (start 94.222999 117.241749) (end 94.86275 117.8815) (width 0.254) (layer B.Cu) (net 3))
 (segment (start 89.149148 126.20625) (end 89.96275 126.20625) (width 0.254) (layer B.Cu) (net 37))
 (segment (start 88.885749 125.942851) (end 89.149148 126.20625) (width 0.254) (layer B.Cu) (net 37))
 (segment (start 88.885749 125.241999) (end 88.885749 125.942851) (width 0.254) (layer B.Cu) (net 37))
 (segment (start 86.51875 122.875) (end 88.885749 125.241999) (width 0.254) (layer B.Cu) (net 37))
 (segment (start 93.10625 119.21875) (end 93.26275 119.37525) (width 0.381) (layer B.Cu) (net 9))
 (segment (start 93.26275 119.37525) (end 93.26275 120.50625) (width 0.381) (layer B.Cu) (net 9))
 (segment (start 87.3125 119.21875) (end 93.10625 119.21875) (width 0.381) (layer B.Cu) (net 9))
 (segment (start 100.9625 133.206) (end 99.66275 131.90625) (width 0.381) (layer B.Cu) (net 9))
 (segment (start 100.9625 134.9375) (end 100.9625 133.206) (width 0.381) (layer B.Cu) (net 9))
 (segment (start 76.6 129.40625) (end 89.96275 129.40625) (width 0.381) (layer B.Cu) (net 9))
 (segment (start 72.23125 125.0375) (end 76.6 129.40625) (width 0.381) (layer B.Cu) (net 9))
 (segment (start 90.4875 133.0815) (end 91.66275 131.90625) (width 0.381) (layer B.Cu) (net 9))
 (segment (start 90.4875 134.9375) (end 90.4875 133.0815) (width 0.381) (layer B.Cu) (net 9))
 (segment (start 104.59375 123.00625) (end 101.36275 123.00625) (width 0.381) (layer B.Cu) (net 9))
 (segment (start 104.775 123.1875) (end 104.59375 123.00625) (width 0.381) (layer B.Cu) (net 9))
 (segment (start 86.125 118.03125) (end 87.3125 119.21875) (width 0.381) (layer B.Cu) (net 9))
 (segment (start 83.34375 118.03125) (end 86.125 118.03125) (width 0.381) (layer B.Cu) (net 9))
 (segment (start 145.034 118.20425) (end 145.034 118.491) (width 0.254) (layer B.Cu) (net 23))
 (segment (start 145.034 118.491) (end 144.681599 118.843401) (width 0.254) (layer B.Cu) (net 23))
 (segment (start 142.875 120.65) (end 128.5875 120.65) (width 0.254) (layer B.Cu) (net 23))
 (segment (start 144.681599 118.843401) (end 142.875 120.65) (width 0.254) (layer B.Cu) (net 23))
 (segment (start 145.034 114.90425) (end 144.273 114.90425) (width 0.254) (layer B.Cu) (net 43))
 (segment (start 141.39125 112.0225) (end 139.7105 112.0225) (width 0.254) (layer B.Cu) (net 43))
 (segment (start 144.273 114.90425) (end 141.39125 112.0225) (width 0.254) (layer B.Cu) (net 43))
 (segment (start 72.23125 118.208982) (end 72.23125 122.2375) (width 0.254) (layer B.Cu) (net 5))
 (segment (start 74.6 115.840232) (end 72.23125 118.208982) (width 0.254) (layer B.Cu) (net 5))
 (segment (start 74.6 113.24375) (end 74.6 115.840232) (width 0.254) (layer B.Cu) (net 5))
 (via (at 80.16875 138.1125) (size 0.8) (drill 0.4) (layers F.Cu B.Cu) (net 31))
 (segment (start 79.6375 138.64375) (end 80.16875 138.1125) (width 0.254) (layer B.Cu) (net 31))
 (segment (start 78.50625 138.64375) (end 79.6375 138.64375) (width 0.254) (layer B.Cu) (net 31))
 (via (at 83.34375 121.44375) (size 0.8) (drill 0.4) (layers F.Cu B.Cu) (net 31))
 (segment (start 83.34375 134.9375) (end 83.34375 121.44375) (width 0.254) (layer F.Cu) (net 31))
 (segment (start 80.16875 138.1125) (end 83.34375 134.9375) (width 0.254) (layer F.Cu) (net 31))
 (segment (start 83.34375 121.44375) (end 83.34375 119.85625) (width 0.254) (layer B.Cu) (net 31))
 (segment (start 92.46275 121.319852) (end 92.46275 120.50625) (width 0.254) (layer B.Cu) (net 31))
 (segment (start 92.178353 121.604249) (end 92.46275 121.319852) (width 0.254) (layer B.Cu) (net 31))
 (segment (start 85.091749 121.604249) (end 92.178353 121.604249) (width 0.254) (layer B.Cu) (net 31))
 (segment (start 83.34375 119.85625) (end 85.091749 121.604249) (width 0.254) (layer B.Cu) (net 31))
 (segment (start 76.2 116.5625) (end 76.99375 117.35625) (width 0.254) (layer B.Cu) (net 7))
 (segment (start 76.2 113.24375) (end 76.2 116.5625) (width 0.254) (layer B.Cu) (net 7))
 (segment (start 89.95025 127.79375) (end 89.96275 127.80625) (width 0.254) (layer B.Cu) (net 38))
 (segment (start 80.16875 127.79375) (end 89.95025 127.79375) (width 0.254) (layer B.Cu) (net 38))
 (segment (start 76.2 123.825) (end 80.16875 127.79375) (width 0.254) (layer B.Cu) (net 38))
 (segment (start 76.2 120.65) (end 76.2 123.825) (width 0.254) (layer B.Cu) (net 38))
 (segment (start 76.99375 119.85625) (end 76.2 120.65) (width 0.254) (layer B.Cu) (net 38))
 (segment (start 76.99375 119.18125) (end 76.99375 119.85625) (width 0.254) (layer B.Cu) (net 38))
 (segment (start 74.60625 117.35) (end 74.6125 117.35625) (width 0.254) (layer B.Cu) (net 6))
 (segment (start 75.4 116.56875) (end 74.6125 117.35625) (width 0.254) (layer B.Cu) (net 6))
 (segment (start 75.4 113.24375) (end 75.4 116.56875) (width 0.254) (layer B.Cu) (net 6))
 (segment (start 74.6125 119.18125) (end 74.6125 119.85625) (width 0.254) (layer B.Cu) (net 39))
 (segment (start 74.6125 119.85625) (end 75.40625 120.65) (width 0.254) (layer B.Cu) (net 39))
 (segment (start 75.40625 120.65) (end 75.40625 123.825) (width 0.254) (layer B.Cu) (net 39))
 (segment (start 80.1875 128.60625) (end 89.96275 128.60625) (width 0.254) (layer B.Cu) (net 39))
 (segment (start 75.40625 123.825) (end 80.1875 128.60625) (width 0.254) (layer B.Cu) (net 39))
 (segment (start 103.98125 131.7625) (end 103.98125 130.96875) (width 0.254) (layer B.Cu) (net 17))
 (segment (start 103.21875 130.20625) (end 101.36275 130.20625) (width 0.254) (layer B.Cu) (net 17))
 (segment (start 103.98125 130.96875) (end 103.21875 130.20625) (width 0.254) (layer B.Cu) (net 17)))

